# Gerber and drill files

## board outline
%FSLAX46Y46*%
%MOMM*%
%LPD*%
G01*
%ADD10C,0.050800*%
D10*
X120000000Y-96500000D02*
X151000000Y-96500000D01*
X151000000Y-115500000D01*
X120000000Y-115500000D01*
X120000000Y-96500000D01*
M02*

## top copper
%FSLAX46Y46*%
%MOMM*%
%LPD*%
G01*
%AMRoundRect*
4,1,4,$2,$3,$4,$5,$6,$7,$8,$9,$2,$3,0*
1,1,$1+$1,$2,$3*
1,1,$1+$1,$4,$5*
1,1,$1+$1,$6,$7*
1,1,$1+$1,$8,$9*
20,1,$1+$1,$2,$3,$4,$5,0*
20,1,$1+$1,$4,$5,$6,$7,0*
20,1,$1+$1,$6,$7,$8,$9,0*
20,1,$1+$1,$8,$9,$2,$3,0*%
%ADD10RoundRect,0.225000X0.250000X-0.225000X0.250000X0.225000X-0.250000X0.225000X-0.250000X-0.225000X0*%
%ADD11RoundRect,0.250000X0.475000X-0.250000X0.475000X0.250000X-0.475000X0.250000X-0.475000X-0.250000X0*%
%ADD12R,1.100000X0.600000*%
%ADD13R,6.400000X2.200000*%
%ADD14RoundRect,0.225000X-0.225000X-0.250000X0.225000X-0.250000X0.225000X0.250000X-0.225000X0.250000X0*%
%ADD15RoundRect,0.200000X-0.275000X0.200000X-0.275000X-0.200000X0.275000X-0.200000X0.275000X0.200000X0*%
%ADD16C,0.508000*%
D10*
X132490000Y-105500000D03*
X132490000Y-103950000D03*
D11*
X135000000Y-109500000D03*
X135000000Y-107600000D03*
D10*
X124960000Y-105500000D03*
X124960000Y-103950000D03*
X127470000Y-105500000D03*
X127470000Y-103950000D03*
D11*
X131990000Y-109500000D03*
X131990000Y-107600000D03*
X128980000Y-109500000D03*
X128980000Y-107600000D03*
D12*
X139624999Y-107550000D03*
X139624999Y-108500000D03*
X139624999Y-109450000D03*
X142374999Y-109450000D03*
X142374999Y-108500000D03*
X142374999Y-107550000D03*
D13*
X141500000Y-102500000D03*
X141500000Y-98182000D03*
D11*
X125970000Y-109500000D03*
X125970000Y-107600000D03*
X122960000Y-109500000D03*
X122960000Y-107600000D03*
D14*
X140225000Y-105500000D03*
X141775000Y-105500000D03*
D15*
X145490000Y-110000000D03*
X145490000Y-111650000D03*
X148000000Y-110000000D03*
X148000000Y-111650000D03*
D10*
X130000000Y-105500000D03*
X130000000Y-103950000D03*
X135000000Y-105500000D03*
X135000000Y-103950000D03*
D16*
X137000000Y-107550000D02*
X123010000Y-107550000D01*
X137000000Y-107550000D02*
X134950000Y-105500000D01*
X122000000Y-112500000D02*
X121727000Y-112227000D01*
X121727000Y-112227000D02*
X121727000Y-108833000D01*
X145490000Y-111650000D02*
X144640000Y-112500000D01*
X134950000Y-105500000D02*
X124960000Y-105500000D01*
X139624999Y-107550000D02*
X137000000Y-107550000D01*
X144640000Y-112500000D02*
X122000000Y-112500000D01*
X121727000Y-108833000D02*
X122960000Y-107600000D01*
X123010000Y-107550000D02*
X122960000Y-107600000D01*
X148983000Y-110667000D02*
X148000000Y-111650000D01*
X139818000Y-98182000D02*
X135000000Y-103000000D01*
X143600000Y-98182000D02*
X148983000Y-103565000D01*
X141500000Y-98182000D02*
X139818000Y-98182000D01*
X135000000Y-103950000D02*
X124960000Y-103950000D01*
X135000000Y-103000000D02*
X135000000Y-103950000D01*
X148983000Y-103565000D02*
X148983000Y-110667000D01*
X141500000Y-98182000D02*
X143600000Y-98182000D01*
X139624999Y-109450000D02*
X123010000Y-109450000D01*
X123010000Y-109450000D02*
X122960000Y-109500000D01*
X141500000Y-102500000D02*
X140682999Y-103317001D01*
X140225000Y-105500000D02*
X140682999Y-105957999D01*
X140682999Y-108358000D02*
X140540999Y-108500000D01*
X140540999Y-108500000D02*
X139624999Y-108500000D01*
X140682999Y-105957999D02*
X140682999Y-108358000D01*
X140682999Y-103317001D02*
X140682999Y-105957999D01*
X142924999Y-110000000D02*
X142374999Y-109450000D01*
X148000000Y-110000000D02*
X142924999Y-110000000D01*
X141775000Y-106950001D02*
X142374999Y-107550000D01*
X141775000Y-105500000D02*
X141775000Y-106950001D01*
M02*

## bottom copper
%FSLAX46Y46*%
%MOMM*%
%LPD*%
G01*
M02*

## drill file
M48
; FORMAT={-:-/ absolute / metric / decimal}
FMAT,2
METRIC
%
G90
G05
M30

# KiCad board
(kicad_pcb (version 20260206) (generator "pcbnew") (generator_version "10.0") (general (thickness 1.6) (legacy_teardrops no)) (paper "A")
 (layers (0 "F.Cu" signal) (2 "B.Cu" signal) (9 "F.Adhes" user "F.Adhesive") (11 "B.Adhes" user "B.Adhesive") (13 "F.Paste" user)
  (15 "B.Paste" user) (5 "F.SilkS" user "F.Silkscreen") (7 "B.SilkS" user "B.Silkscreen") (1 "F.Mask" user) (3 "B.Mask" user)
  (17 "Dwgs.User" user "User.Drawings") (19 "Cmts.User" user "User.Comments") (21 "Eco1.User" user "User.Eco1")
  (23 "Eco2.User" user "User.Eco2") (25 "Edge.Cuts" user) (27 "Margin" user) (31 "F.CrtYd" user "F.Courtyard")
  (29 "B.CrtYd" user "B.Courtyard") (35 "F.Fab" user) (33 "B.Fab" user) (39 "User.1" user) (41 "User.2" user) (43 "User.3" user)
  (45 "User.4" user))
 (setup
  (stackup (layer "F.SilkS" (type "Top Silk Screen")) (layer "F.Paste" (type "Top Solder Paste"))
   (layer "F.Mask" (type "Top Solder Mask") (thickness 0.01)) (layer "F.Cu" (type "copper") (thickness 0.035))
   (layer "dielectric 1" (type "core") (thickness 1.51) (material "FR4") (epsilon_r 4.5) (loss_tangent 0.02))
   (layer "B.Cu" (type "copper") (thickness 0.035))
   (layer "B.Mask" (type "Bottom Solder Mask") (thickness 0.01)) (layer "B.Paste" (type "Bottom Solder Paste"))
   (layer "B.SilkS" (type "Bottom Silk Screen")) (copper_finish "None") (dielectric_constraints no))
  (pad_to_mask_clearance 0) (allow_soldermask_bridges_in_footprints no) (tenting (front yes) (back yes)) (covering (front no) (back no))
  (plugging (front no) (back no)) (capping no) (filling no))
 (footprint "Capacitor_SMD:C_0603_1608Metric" (layer "F.Cu") (at 132.49 104.725 90)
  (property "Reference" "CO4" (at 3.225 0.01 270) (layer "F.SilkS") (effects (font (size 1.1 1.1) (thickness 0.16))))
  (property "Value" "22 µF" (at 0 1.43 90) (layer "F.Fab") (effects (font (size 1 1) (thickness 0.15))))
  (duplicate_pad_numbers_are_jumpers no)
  (pad "1" smd roundrect (at -0.775 0 90) (size 0.9 0.95) (layers "F.Cu" "F.Mask" "F.Paste") (roundrect_rratio 0.25) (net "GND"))
  (pad "2" smd roundrect (at 0.775 0 90) (size 0.9 0.95) (layers "F.Cu" "F.Mask" "F.Paste") (roundrect_rratio 0.25) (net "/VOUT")))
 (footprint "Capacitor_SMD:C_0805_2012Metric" (layer "F.Cu") (at 135 108.55 90)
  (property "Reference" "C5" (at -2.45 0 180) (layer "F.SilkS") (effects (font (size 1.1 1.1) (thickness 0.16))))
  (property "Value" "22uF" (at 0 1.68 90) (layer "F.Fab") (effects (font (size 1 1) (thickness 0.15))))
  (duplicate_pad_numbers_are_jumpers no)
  (pad "1" smd roundrect (at -0.95 0 90) (size 1 1.45) (layers "F.Cu" "F.Mask" "F.Paste") (roundrect_rratio 0.25) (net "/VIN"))
  (pad "2" smd roundrect (at 0.95 0 90) (size 1 1.45) (layers "F.Cu" "F.Mask" "F.Paste") (roundrect_rratio 0.25) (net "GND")))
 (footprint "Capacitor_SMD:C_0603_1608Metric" (layer "F.Cu") (at 124.96 104.725 90)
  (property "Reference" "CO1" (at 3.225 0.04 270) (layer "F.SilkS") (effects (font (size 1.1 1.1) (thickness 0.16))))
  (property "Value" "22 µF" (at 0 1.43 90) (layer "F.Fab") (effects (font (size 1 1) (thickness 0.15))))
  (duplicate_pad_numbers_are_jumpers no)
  (pad "1" smd roundrect (at -0.775 0 90) (size 0.9 0.95) (layers "F.Cu" "F.Mask" "F.Paste") (roundrect_rratio 0.25) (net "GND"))
  (pad "2" smd roundrect (at 0.775 0 90) (size 0.9 0.95) (layers "F.Cu" "F.Mask" "F.Paste") (roundrect_rratio 0.25) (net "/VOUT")))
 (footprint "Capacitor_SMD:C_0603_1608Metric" (layer "F.Cu") (at 127.47 104.725 90)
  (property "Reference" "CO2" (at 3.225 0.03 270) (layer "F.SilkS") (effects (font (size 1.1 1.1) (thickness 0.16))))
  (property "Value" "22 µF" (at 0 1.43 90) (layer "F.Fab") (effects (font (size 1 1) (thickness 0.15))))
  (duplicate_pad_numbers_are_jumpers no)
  (pad "1" smd roundrect (at -0.775 0 90) (size 0.9 0.95) (layers "F.Cu" "F.Mask" "F.Paste") (roundrect_rratio 0.25) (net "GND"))
  (pad "2" smd roundrect (at 0.775 0 90) (size 0.9 0.95) (layers "F.Cu" "F.Mask" "F.Paste") (roundrect_rratio 0.25) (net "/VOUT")))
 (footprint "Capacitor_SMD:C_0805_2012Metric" (layer "F.Cu") (at 131.99 108.55 90)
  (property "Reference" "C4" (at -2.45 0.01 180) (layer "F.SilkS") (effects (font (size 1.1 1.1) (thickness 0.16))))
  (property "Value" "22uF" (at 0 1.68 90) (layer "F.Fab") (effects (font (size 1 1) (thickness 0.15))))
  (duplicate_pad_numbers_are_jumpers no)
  (pad "1" smd roundrect (at -0.95 0 90) (size 1 1.45) (layers "F.Cu" "F.Mask" "F.Paste") (roundrect_rratio 0.25) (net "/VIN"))
  (pad "2" smd roundrect (at 0.95 0 90) (size 1 1.45) (layers "F.Cu" "F.Mask" "F.Paste") (roundrect_rratio 0.25) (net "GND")))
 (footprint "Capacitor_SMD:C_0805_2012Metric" (layer "F.Cu") (at 128.98 108.55 90)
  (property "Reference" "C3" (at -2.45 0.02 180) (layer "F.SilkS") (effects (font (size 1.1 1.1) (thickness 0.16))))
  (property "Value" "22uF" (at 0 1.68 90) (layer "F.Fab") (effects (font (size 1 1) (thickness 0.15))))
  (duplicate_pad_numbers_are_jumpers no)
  (pad "1" smd roundrect (at -0.95 0 90) (size 1 1.45) (layers "F.Cu" "F.Mask" "F.Paste") (roundrect_rratio 0.25) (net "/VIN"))
  (pad "2" smd roundrect (at 0.95 0 90) (size 1 1.45) (layers "F.Cu" "F.Mask" "F.Paste") (roundrect_rratio 0.25) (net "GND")))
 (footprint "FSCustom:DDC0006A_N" (layer "F.Cu") (at 141 108.5)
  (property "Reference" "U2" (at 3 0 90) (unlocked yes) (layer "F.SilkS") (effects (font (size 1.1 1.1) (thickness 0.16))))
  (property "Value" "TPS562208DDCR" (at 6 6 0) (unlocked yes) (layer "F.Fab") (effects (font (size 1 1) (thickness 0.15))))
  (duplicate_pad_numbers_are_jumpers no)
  (pad "1" smd rect (at -1.375001 -0.95 90) (size 0.6 1.1) (layers "F.Cu" "F.Mask" "F.Paste") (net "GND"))
  (pad "2" smd rect (at -1.375001 0 90) (size 0.6 1.1) (layers "F.Cu" "F.Mask" "F.Paste") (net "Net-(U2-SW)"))
  (pad "3" smd rect (at -1.375001 0.95 90) (size 0.6 1.1) (layers "F.Cu" "F.Mask" "F.Paste") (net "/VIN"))
  (pad "4" smd rect (at 1.374999 0.95 90) (size 0.6 1.1) (layers "F.Cu" "F.Mask" "F.Paste") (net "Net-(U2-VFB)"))
  (pad "5" smd rect (at 1.374999 0 90) (size 0.6 1.1) (layers "F.Cu" "F.Mask" "F.Paste") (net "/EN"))
  (pad "6" smd rect (at 1.374999 -0.95 90) (size 0.6 1.1) (layers "F.Cu" "F.Mask" "F.Paste") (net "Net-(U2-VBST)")))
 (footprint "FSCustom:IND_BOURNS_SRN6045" (layer "F.Cu") (at 141.5 100.341 90)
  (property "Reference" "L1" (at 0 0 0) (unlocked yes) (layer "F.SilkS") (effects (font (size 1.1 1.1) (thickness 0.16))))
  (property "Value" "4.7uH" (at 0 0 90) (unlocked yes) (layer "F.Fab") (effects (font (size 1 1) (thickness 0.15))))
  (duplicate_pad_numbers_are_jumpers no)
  (pad "1" smd rect (at -2.159 0 90) (size 2.2 6.4) (layers "F.Cu" "F.Mask" "F.Paste") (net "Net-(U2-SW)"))
  (pad "2" smd rect (at 2.159 0 90) (size 2.2 6.4) (layers "F.Cu" "F.Mask" "F.Paste") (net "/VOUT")))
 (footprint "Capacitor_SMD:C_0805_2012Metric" (layer "F.Cu") (at 125.97 108.55 90)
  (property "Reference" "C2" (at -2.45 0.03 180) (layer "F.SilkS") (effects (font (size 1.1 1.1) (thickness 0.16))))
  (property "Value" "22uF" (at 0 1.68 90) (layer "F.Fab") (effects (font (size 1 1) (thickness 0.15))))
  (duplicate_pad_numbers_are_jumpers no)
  (pad "1" smd roundrect (at -0.95 0 90) (size 1 1.45) (layers "F.Cu" "F.Mask" "F.Paste") (roundrect_rratio 0.25) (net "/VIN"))
  (pad "2" smd roundrect (at 0.95 0 90) (size 1 1.45) (layers "F.Cu" "F.Mask" "F.Paste") (roundrect_rratio 0.25) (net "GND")))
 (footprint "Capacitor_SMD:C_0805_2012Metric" (layer "F.Cu") (at 122.96 108.55 90)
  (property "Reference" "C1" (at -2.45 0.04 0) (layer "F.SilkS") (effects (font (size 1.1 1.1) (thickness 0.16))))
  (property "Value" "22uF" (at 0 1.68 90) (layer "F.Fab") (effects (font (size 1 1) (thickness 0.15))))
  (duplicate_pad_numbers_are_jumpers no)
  (pad "1" smd roundrect (at -0.95 0 90) (size 1 1.45) (layers "F.Cu" "F.Mask" "F.Paste") (roundrect_rratio 0.25) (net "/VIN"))
  (pad "2" smd roundrect (at 0.95 0 90) (size 1 1.45) (layers "F.Cu" "F.Mask" "F.Paste") (roundrect_rratio 0.25) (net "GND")))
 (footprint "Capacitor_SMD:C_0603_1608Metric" (layer "F.Cu") (at 141 105.5)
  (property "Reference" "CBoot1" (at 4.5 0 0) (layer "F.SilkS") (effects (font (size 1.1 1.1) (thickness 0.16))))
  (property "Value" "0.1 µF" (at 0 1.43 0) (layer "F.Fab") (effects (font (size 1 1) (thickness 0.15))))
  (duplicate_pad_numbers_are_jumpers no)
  (pad "1" smd roundrect (at -0.775 0) (size 0.9 0.95) (layers "F.Cu" "F.Mask" "F.Paste") (roundrect_rratio 0.25) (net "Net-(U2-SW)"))
  (pad "2" smd roundrect (at 0.775 0) (size 0.9 0.95) (layers "F.Cu" "F.Mask" "F.Paste") (roundrect_rratio 0.25) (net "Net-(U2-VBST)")))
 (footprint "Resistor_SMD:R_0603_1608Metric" (layer "F.Cu") (at 145.49 110.825 -90)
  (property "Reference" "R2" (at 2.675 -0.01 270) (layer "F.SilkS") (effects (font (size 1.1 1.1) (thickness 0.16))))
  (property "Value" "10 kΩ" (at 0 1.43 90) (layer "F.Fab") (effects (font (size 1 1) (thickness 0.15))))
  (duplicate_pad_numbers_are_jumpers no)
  (pad "1" smd roundrect (at -0.825 0 270) (size 0.8 0.95) (layers "F.Cu" "F.Mask" "F.Paste") (roundrect_rratio 0.25) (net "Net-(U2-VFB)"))
  (pad "2" smd roundrect (at 0.825 0 270) (size 0.8 0.95) (layers "F.Cu" "F.Mask" "F.Paste") (roundrect_rratio 0.25) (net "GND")))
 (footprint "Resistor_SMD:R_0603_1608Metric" (layer "F.Cu") (at 148 110.825 -90)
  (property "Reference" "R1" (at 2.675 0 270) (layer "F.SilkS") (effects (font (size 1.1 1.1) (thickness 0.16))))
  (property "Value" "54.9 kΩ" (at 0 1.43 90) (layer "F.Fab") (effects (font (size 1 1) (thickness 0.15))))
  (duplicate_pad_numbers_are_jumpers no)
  (pad "1" smd roundrect (at -0.825 0 270) (size 0.8 0.95) (layers "F.Cu" "F.Mask" "F.Paste") (roundrect_rratio 0.25) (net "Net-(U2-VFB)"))
  (pad "2" smd roundrect (at 0.825 0 270) (size 0.8 0.95) (layers "F.Cu" "F.Mask" "F.Paste") (roundrect_rratio 0.25) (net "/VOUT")))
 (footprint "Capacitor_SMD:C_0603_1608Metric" (layer "F.Cu") (at 130 104.725 90)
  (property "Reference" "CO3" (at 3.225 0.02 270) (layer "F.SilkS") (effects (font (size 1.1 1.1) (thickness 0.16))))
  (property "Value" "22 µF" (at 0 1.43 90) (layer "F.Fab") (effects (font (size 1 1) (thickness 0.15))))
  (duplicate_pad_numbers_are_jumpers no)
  (pad "1" smd roundrect (at -0.775 0 90) (size 0.9 0.95) (layers "F.Cu" "F.Mask" "F.Paste") (roundrect_rratio 0.25) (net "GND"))
  (pad "2" smd roundrect (at 0.775 0 90) (size 0.9 0.95) (layers "F.Cu" "F.Mask" "F.Paste") (roundrect_rratio 0.25) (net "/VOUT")))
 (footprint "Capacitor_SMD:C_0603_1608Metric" (layer "F.Cu") (at 135 104.725 90)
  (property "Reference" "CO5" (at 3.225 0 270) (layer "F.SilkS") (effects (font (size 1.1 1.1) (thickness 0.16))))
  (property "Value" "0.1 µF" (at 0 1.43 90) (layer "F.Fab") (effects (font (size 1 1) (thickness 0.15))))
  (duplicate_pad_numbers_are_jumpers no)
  (pad "1" smd roundrect (at -0.775 0 90) (size 0.9 0.95) (layers "F.Cu" "F.Mask" "F.Paste") (roundrect_rratio 0.25) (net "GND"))
  (pad "2" smd roundrect (at 0.775 0 90) (size 0.9 0.95) (layers "F.Cu" "F.Mask" "F.Paste") (roundrect_rratio 0.25) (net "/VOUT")))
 (gr_rect (start 120 96.5) (end 151 115.5) (stroke (width 0.0508) (type default)) (fill no) (layer "Edge.Cuts"))
 (segment (start 137 107.55) (end 123.01 107.55) (width 0.508) (layer "F.Cu") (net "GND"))
 (segment (start 137 107.55) (end 134.95 105.5) (width 0.508) (layer "F.Cu") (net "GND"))
 (segment (start 122 112.5) (end 121.727 112.227) (width 0.508) (layer "F.Cu") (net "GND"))
 (segment (start 121.727 112.227) (end 121.727 108.833) (width 0.508) (layer "F.Cu") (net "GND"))
 (segment (start 145.49 111.65) (end 144.64 112.5) (width 0.508) (layer "F.Cu") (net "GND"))
 (segment (start 134.95 105.5) (end 124.96 105.5) (width 0.508) (layer "F.Cu") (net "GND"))
 (segment (start 139.624999 107.55) (end 137 107.55) (width 0.508) (layer "F.Cu") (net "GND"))
 (segment (start 144.64 112.5) (end 122 112.5) (width 0.508) (layer "F.Cu") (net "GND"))
 (segment (start 121.727 108.833) (end 122.96 107.6) (width 0.508) (layer "F.Cu") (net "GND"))
 (segment (start 123.01 107.55) (end 122.96 107.6) (width 0.508) (layer "F.Cu") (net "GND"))
 (segment (start 148.983 110.667) (end 148 111.65) (width 0.508) (layer "F.Cu") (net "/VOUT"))
 (segment (start 139.818 98.182) (end 135 103) (width 0.508) (layer "F.Cu") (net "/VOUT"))
 (segment (start 143.6 98.182) (end 148.983 103.565) (width 0.508) (layer "F.Cu") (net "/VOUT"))
 (segment (start 141.5 98.182) (end 139.818 98.182) (width 0.508) (layer "F.Cu") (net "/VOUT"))
 (segment (start 135 103.95) (end 124.96 103.95) (width 0.508) (layer "F.Cu") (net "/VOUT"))
 (segment (start 135 103) (end 135 103.95) (width 0.508) (layer "F.Cu") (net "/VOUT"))
 (segment (start 148.983 103.565) (end 148.983 110.667) (width 0.508) (layer "F.Cu") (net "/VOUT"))
 (segment (start 141.5 98.182) (end 143.6 98.182) (width 0.508) (layer "F.Cu") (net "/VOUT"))
 (segment (start 139.624999 109.45) (end 123.01 109.45) (width 0.508) (layer "F.Cu") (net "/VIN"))
 (segment (start 123.01 109.45) (end 122.96 109.5) (width 0.508) (layer "F.Cu") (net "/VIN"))
 (segment (start 141.5 102.5) (end 140.682999 103.317001) (width 0.508) (layer "F.Cu") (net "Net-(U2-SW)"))
 (segment (start 140.225 105.5) (end 140.682999 105.957999) (width 0.508) (layer "F.Cu") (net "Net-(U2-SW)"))
 (segment (start 140.682999 108.358) (end 140.540999 108.5) (width 0.508) (layer "F.Cu") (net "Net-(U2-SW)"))
 (segment (start 140.540999 108.5) (end 139.624999 108.5) (width 0.508) (layer "F.Cu") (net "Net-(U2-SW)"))
 (segment (start 140.682999 105.957999) (end 140.682999 108.358) (width 0.508) (layer "F.Cu") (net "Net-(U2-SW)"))
 (segment (start 140.682999 103.317001) (end 140.682999 105.957999) (width 0.508) (layer "F.Cu") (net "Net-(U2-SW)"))
 (segment (start 142.924999 110) (end 142.374999 109.45) (width 0.508) (layer "F.Cu") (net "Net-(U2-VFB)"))
 (segment (start 148 110) (end 142.924999 110) (width 0.508) (layer "F.Cu") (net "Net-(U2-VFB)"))
 (segment (start 141.775 106.950001) (end 142.374999 107.55) (width 0.508) (layer "F.Cu") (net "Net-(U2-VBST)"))
 (segment (start 141.775 105.5) (end 141.775 106.950001) (width 0.508) (layer "F.Cu") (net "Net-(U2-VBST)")))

